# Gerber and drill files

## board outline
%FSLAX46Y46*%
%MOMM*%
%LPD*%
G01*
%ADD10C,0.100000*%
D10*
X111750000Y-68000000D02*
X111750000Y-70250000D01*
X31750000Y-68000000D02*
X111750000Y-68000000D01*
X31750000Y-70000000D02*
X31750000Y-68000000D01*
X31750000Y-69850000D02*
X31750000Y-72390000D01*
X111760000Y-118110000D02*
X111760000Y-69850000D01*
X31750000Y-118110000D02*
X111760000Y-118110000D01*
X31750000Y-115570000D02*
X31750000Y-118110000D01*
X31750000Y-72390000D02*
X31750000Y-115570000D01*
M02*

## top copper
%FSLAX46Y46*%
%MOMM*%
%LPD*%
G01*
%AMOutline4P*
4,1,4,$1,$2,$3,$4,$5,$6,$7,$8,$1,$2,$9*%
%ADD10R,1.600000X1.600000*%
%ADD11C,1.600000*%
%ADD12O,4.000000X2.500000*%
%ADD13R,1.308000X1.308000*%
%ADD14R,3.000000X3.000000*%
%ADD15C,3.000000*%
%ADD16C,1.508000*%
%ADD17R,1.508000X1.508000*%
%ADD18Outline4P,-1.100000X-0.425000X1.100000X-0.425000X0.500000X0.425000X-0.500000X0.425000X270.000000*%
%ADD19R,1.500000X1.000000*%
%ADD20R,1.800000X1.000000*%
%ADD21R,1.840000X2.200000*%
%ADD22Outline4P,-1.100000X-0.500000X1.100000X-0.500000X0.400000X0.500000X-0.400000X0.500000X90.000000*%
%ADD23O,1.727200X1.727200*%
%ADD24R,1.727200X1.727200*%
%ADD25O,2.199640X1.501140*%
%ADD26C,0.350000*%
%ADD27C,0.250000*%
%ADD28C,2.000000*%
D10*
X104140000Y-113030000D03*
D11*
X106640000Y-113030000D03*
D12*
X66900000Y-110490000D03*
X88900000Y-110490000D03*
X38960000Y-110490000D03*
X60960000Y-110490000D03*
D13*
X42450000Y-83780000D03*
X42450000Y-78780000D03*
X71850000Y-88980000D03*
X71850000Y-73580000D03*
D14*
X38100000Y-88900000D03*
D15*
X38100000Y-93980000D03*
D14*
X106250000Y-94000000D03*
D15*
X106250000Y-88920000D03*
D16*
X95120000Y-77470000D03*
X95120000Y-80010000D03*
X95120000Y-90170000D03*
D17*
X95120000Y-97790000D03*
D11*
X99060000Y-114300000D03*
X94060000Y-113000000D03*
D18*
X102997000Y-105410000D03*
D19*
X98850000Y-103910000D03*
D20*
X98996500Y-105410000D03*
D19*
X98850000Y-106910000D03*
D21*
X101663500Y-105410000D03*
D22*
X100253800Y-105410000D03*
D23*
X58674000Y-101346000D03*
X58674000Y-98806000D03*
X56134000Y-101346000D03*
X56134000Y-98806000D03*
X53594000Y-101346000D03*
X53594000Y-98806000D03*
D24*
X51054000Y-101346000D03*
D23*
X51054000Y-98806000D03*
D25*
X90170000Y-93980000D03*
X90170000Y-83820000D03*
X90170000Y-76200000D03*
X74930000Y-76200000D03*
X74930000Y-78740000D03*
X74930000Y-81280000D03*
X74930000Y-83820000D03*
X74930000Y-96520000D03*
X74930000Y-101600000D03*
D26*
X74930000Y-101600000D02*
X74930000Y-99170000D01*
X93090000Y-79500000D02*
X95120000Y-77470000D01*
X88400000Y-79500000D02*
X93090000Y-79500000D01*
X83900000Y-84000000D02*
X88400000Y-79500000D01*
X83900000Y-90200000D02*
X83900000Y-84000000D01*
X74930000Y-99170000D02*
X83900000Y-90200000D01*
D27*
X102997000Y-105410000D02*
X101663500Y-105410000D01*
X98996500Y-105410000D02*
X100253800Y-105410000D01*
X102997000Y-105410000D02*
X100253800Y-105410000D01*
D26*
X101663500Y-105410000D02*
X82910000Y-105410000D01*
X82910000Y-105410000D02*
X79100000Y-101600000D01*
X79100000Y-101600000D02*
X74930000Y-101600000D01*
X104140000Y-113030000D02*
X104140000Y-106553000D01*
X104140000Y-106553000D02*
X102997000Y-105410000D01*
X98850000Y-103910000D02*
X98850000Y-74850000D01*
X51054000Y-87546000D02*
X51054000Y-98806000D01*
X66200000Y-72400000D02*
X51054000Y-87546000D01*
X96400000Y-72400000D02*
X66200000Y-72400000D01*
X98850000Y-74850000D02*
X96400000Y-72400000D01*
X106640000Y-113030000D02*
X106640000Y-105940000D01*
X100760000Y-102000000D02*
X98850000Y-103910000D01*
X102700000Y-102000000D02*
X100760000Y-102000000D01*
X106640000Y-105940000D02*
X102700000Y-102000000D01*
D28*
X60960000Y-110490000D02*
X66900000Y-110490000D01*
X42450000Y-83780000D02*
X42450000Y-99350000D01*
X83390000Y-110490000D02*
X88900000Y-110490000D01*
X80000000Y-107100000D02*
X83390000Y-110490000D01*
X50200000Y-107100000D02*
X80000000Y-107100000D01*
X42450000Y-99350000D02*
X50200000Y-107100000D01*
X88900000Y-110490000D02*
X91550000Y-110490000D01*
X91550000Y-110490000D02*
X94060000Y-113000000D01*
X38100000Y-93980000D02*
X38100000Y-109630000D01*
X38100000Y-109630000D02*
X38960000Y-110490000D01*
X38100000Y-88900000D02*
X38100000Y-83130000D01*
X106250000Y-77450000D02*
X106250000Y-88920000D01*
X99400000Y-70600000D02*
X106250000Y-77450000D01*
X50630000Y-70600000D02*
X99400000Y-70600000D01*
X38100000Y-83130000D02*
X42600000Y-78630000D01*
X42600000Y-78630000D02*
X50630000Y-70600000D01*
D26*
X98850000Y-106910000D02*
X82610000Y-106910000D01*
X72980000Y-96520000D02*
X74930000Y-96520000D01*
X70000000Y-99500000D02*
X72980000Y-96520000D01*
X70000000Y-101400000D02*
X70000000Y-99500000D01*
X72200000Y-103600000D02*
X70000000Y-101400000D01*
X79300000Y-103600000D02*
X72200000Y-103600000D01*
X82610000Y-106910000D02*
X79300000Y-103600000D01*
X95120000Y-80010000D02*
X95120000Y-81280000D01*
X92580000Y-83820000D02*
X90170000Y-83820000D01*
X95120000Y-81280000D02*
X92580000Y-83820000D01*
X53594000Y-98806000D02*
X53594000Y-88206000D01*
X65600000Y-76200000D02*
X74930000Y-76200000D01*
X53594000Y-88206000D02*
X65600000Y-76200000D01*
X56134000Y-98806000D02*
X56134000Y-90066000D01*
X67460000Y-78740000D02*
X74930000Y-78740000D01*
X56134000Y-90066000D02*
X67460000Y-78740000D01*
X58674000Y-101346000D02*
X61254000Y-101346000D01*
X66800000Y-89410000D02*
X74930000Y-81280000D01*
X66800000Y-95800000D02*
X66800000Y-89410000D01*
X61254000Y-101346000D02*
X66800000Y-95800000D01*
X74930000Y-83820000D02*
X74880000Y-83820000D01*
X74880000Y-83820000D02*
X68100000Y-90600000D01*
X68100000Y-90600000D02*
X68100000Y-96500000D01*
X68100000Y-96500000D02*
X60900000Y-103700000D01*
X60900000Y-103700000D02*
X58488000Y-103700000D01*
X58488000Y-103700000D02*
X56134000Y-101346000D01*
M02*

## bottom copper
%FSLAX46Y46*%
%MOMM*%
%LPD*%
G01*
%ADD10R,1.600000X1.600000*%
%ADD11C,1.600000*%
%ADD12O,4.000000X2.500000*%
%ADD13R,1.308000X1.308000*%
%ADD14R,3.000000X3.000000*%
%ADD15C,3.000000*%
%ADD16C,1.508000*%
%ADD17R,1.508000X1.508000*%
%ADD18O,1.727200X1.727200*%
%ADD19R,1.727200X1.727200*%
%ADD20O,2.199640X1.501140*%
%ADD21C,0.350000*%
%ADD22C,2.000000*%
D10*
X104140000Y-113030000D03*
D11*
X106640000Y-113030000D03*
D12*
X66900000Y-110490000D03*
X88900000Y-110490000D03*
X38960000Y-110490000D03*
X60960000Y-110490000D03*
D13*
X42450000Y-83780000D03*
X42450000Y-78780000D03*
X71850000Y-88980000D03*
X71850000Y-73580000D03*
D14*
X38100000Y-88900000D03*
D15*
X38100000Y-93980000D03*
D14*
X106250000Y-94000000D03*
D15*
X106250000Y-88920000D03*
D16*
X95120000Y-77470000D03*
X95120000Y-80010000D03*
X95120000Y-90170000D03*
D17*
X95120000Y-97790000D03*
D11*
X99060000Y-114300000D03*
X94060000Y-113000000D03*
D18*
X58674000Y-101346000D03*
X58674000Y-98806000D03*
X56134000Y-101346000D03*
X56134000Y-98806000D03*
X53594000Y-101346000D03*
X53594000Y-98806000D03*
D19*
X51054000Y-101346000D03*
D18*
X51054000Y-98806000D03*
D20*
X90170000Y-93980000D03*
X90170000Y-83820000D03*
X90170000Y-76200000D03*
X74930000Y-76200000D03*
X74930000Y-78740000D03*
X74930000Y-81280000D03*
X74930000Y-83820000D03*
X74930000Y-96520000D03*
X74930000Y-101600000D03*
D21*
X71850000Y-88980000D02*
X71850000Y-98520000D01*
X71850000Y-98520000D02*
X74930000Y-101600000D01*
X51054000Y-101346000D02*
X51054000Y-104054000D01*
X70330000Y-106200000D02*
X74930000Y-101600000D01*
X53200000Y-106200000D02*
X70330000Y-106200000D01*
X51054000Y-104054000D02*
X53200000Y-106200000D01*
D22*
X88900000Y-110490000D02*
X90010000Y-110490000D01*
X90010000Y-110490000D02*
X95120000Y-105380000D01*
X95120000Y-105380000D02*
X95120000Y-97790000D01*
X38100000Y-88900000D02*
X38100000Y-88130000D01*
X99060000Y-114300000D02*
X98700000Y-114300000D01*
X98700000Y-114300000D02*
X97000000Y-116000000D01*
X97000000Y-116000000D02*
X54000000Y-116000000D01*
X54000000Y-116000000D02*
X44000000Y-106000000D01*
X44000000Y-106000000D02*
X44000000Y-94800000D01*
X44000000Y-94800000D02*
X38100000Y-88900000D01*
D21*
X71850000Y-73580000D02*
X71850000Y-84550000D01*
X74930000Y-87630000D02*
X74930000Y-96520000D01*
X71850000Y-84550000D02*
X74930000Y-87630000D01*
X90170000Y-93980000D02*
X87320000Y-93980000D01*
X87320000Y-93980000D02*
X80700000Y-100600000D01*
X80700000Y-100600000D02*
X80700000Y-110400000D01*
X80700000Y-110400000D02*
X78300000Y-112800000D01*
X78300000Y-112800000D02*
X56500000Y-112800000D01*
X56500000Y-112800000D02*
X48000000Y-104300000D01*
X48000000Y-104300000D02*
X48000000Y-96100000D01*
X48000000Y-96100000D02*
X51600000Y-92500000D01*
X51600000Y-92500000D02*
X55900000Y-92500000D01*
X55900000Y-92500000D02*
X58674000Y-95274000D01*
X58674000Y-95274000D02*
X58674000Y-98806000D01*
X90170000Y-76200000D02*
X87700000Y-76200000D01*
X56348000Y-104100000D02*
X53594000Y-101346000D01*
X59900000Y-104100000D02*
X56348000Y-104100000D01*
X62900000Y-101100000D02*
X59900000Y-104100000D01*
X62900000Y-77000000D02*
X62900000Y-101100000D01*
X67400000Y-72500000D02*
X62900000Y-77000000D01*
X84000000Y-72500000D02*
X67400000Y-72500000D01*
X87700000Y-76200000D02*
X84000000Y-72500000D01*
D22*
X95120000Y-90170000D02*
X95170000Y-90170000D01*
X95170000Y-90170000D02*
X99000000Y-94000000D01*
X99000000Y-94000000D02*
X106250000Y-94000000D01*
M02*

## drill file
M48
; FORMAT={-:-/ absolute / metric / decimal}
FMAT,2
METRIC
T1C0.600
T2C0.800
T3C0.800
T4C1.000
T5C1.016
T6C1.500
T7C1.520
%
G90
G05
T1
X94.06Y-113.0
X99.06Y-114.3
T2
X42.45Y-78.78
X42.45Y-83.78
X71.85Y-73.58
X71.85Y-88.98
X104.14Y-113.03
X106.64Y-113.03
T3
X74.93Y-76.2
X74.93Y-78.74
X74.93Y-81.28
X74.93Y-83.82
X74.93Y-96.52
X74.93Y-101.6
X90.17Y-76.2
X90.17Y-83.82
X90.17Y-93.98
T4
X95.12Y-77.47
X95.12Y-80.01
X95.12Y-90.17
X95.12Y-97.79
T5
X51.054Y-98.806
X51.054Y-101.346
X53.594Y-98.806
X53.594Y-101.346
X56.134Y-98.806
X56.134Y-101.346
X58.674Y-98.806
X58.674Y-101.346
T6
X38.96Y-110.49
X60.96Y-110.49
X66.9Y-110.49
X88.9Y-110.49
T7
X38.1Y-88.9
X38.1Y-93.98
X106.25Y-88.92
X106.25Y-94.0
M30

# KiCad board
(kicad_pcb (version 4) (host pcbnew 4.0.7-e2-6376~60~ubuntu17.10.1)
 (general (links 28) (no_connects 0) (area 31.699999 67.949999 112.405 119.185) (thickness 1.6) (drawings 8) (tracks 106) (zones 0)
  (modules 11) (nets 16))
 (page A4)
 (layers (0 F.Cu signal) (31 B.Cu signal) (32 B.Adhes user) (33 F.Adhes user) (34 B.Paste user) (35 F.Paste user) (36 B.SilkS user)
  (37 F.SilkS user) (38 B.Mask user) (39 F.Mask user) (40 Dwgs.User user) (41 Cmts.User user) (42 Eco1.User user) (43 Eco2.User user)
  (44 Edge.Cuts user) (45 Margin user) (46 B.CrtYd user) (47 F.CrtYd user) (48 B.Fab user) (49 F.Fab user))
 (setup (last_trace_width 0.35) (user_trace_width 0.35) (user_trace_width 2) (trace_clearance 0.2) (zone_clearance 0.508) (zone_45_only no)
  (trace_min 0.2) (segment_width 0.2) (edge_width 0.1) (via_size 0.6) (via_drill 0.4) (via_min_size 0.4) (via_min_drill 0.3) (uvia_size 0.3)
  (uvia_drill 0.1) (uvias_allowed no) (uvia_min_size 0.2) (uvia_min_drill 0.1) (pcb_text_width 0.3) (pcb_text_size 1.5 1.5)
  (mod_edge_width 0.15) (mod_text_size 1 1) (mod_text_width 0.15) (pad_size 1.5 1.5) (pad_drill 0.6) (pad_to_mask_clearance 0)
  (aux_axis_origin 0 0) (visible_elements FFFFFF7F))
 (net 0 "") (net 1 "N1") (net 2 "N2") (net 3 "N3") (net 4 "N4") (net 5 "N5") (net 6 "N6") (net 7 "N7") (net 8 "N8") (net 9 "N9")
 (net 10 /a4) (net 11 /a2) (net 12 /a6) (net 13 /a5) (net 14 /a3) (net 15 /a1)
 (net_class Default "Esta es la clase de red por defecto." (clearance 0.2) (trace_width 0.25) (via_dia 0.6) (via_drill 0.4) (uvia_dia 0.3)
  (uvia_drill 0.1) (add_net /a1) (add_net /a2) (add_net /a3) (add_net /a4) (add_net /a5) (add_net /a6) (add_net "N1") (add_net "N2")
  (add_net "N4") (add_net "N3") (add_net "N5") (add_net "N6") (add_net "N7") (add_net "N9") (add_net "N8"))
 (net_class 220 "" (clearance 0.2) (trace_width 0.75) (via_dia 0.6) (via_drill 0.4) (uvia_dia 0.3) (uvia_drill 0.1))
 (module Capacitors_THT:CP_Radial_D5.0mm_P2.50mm (layer F.Cu) (at 104.14 113.03)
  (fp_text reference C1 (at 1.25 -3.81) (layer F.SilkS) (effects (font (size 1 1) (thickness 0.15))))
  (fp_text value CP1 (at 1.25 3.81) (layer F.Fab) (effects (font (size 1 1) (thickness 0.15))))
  (pad 1 thru_hole rect (at 0 0) (size 1.6 1.6) (drill 0.8) (layers *.Cu *.Mask) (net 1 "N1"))
  (pad 2 thru_hole circle (at 2.5 0) (size 1.6 1.6) (drill 0.8) (layers *.Cu *.Mask) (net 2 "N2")))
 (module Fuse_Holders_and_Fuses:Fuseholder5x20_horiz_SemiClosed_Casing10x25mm (layer F.Cu) (at 88.9 110.49 180)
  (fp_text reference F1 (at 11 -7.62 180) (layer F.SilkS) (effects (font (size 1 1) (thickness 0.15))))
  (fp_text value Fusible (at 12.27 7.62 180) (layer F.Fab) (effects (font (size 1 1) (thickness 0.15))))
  (pad 2 thru_hole oval (at 22 0 90) (size 2.5 4) (drill 1.5) (layers *.Cu *.Mask) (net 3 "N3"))
  (pad 1 thru_hole oval (at 0 0 90) (size 2.5 4) (drill 1.5) (layers *.Cu *.Mask) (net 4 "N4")))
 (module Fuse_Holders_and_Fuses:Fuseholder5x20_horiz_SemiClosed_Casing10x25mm (layer F.Cu) (at 60.96 110.49 180)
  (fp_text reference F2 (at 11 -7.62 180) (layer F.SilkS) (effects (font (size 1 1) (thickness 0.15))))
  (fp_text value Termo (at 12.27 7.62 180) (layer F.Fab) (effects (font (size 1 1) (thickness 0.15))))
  (pad 2 thru_hole oval (at 22 0 90) (size 2.5 4) (drill 1.5) (layers *.Cu *.Mask) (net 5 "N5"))
  (pad 1 thru_hole oval (at 0 0 90) (size 2.5 4) (drill 1.5) (layers *.Cu *.Mask) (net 3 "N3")))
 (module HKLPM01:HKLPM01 (layer B.Cu) (at 57.15 81.28)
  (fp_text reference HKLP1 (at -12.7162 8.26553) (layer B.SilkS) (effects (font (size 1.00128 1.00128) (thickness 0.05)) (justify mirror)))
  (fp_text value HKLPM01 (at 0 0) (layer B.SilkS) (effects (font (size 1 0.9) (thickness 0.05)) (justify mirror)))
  (pad P$1 thru_hole rect (at -14.7 2.5) (size 1.308 1.308) (drill 0.8) (layers *.Cu *.Mask B.SilkS) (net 4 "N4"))
  (pad P$2 thru_hole rect (at -14.7 -2.5) (size 1.308 1.308) (drill 0.8) (layers *.Cu *.Mask B.SilkS) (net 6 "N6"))
  (pad P$3 thru_hole rect (at 14.7 7.7) (size 1.308 1.308) (drill 0.8) (layers *.Cu *.Mask B.SilkS) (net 1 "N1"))
  (pad P$4 thru_hole rect (at 14.7 -7.7) (size 1.308 1.308) (drill 0.8) (layers *.Cu *.Mask B.SilkS) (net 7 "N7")))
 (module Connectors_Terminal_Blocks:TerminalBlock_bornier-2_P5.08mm (layer F.Cu) (at 38.1 88.9 270)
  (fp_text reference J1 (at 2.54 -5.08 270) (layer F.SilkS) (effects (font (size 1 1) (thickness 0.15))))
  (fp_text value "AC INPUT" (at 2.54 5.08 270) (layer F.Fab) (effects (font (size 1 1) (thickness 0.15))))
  (pad 1 thru_hole rect (at 0 0 270) (size 3 3) (drill 1.52) (layers *.Cu *.Mask) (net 6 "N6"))
  (pad 2 thru_hole circle (at 5.08 0 270) (size 3 3) (drill 1.52) (layers *.Cu *.Mask) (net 5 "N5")))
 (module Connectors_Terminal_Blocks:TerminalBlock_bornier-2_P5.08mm (layer F.Cu) (at 106.25 94 90)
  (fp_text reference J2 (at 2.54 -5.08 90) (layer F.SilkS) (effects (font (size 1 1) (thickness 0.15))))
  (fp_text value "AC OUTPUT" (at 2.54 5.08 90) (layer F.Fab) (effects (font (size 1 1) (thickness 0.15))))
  (pad 1 thru_hole rect (at 0 0 90) (size 3 3) (drill 1.52) (layers *.Cu *.Mask) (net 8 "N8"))
  (pad 2 thru_hole circle (at 5.08 0 90) (size 3 3) (drill 1.52) (layers *.Cu *.Mask) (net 6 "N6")))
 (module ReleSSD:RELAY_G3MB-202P (layer F.Cu) (at 96.52 87.63 270)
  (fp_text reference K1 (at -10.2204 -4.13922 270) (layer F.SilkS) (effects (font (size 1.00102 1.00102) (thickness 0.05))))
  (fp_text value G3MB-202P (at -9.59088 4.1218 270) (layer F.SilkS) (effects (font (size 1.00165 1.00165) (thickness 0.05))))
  (pad 4 thru_hole circle (at -10.16 1.4 270) (size 1.508 1.508) (drill 1) (layers *.Cu *.Mask F.SilkS) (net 1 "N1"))
  (pad 3 thru_hole circle (at -7.62 1.4 270) (size 1.508 1.508) (drill 1) (layers *.Cu *.Mask F.SilkS) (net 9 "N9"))
  (pad 2 thru_hole circle (at 2.54 1.4 270) (size 1.508 1.508) (drill 1) (layers *.Cu *.Mask F.SilkS) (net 8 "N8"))
  (pad 1 thru_hole rect (at 10.16 1.4 270) (size 1.508 1.508) (drill 1) (layers *.Cu *.Mask F.SilkS) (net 4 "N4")))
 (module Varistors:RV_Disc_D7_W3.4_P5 (layer F.Cu) (at 99.06 114.3 180)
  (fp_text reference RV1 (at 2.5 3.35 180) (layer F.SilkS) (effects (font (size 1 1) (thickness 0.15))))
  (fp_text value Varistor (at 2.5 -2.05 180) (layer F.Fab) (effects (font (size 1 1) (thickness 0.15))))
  (pad 1 thru_hole circle (at 0 0 180) (size 1.6 1.6) (drill 0.6) (layers *.Cu *.Mask) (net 6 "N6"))
  (pad 2 thru_hole circle (at 5 1.3 180) (size 1.6 1.6) (drill 0.6) (layers *.Cu *.Mask) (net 4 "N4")))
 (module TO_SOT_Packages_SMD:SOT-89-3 (layer F.Cu) (at 100.33 105.41)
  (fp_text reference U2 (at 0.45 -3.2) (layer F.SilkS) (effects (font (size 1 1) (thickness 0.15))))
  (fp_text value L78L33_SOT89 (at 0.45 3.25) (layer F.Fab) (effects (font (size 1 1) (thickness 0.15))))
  (pad 2 smd trapezoid (at 2.667 0 270) (size 1.6 0.85) (rect_delta 0 0.6) (layers F.Cu F.Paste F.Mask) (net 1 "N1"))
  (pad 1 smd rect (at -1.48 -1.5 270) (size 1 1.5) (layers F.Cu F.Paste F.Mask) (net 2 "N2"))
  (pad 2 smd rect (at -1.3335 0 270) (size 1 1.8) (layers F.Cu F.Paste F.Mask) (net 1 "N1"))
  (pad 3 smd rect (at -1.48 1.5 270) (size 1 1.5) (layers F.Cu F.Paste F.Mask) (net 7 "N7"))
  (pad 2 smd rect (at 1.3335 0 270) (size 2.2 1.84) (layers F.Cu F.Paste F.Mask) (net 1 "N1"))
  (pad 2 smd trapezoid (at -0.0762 0 90) (size 1.5 1) (rect_delta 0 0.7) (layers F.Cu F.Paste F.Mask) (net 1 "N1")))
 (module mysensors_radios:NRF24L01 (layer F.Cu) (at 49.53 102.87 180)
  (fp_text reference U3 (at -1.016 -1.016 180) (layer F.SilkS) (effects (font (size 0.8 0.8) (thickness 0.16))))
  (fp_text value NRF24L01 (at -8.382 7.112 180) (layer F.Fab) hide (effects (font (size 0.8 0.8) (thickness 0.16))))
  (pad 7 thru_hole oval (at -9.144 1.524 180) (size 1.7272 1.7272) (drill 1.016) (layers *.Cu *.Mask F.SilkS) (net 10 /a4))
  (pad 8 thru_hole oval (at -9.144 4.064 180) (size 1.7272 1.7272) (drill 1.016) (layers *.Cu *.Mask F.SilkS) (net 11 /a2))
  (pad 5 thru_hole oval (at -6.604 1.524 180) (size 1.7272 1.7272) (drill 1.016) (layers *.Cu *.Mask F.SilkS) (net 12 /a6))
  (pad 6 thru_hole oval (at -6.604 4.064 180) (size 1.7272 1.7272) (drill 1.016) (layers *.Cu *.Mask F.SilkS) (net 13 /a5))
  (pad 3 thru_hole oval (at -4.064 1.524 180) (size 1.7272 1.7272) (drill 1.016) (layers *.Cu *.Mask F.SilkS) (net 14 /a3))
  (pad 4 thru_hole oval (at -4.064 4.064 180) (size 1.7272 1.7272) (drill 1.016) (layers *.Cu *.Mask F.SilkS) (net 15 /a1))
  (pad 1 thru_hole rect (at -1.524 1.524 180) (size 1.7272 1.7272) (drill 1.016) (layers *.Cu *.Mask F.SilkS) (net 1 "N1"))
  (pad 2 thru_hole oval (at -1.524 4.064 180) (size 1.7272 1.7272) (drill 1.016) (layers *.Cu *.Mask F.SilkS) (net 2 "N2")))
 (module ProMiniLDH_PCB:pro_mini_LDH (layer F.Cu) (at 82.55 90.17 90)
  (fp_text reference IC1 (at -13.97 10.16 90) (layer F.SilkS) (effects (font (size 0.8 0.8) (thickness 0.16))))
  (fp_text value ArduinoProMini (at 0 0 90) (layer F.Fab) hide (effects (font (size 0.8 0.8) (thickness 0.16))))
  (pad 5 thru_hole oval (at -3.81 7.62 90) (size 1.50114 2.19964) (drill 0.8001) (layers *.Cu *.Mask F.SilkS) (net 11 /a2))
  (pad 9 thru_hole oval (at 6.35 7.62 90) (size 1.50114 2.19964) (drill 0.8001) (layers *.Cu *.Mask F.SilkS) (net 9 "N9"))
  (pad 12 thru_hole oval (at 13.97 7.62 90) (size 1.50114 2.19964) (drill 0.8001) (layers *.Cu *.Mask F.SilkS) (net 14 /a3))
  (pad 13 thru_hole oval (at 13.97 -7.62 90) (size 1.50114 2.19964) (drill 0.8001) (layers *.Cu *.Mask F.SilkS) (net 15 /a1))
  (pad 14 thru_hole oval (at 11.43 -7.62 90) (size 1.50114 2.19964) (drill 0.8001) (layers *.Cu *.Mask F.SilkS) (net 13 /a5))
  (pad 15 thru_hole oval (at 8.89 -7.62 90) (size 1.50114 2.19964) (drill 0.8001) (layers *.Cu *.Mask F.SilkS) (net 10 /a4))
  (pad 16 thru_hole oval (at 6.35 -7.62 90) (size 1.50114 2.19964) (drill 0.8001) (layers *.Cu *.Mask F.SilkS) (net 12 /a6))
  (pad 21 thru_hole oval (at -6.35 -7.62 90) (size 1.50114 2.19964) (drill 0.8001) (layers *.Cu *.Mask F.SilkS) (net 7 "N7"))
  (pad 23 thru_hole oval (at -11.43 -7.62 90) (size 1.50114 2.19964) (drill 0.8001) (layers *.Cu *.Mask F.SilkS) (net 1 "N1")))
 (gr_line (start 111.75 68) (end 111.75 70.25) (angle 90) (layer Edge.Cuts) (width 0.1))
 (gr_line (start 31.75 68) (end 111.75 68) (angle 90) (layer Edge.Cuts) (width 0.1))
 (gr_line (start 31.75 70) (end 31.75 68) (angle 90) (layer Edge.Cuts) (width 0.1))
 (gr_line (start 31.75 69.85) (end 31.75 72.39) (angle 90) (layer Edge.Cuts) (width 0.1))
 (gr_line (start 111.76 118.11) (end 111.76 69.85) (angle 90) (layer Edge.Cuts) (width 0.1))
 (gr_line (start 31.75 118.11) (end 111.76 118.11) (angle 90) (layer Edge.Cuts) (width 0.1))
 (gr_line (start 31.75 115.57) (end 31.75 118.11) (angle 90) (layer Edge.Cuts) (width 0.1))
 (gr_line (start 31.75 72.39) (end 31.75 115.57) (angle 90) (layer Edge.Cuts) (width 0.1))
 (segment (start 74.93 101.6) (end 74.93 99.17) (width 0.35) (layer F.Cu) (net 1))
 (segment (start 93.09 79.5) (end 95.12 77.47) (width 0.35) (layer F.Cu) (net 1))
 (segment (start 88.4 79.5) (end 93.09 79.5) (width 0.35) (layer F.Cu) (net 1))
 (segment (start 83.9 84) (end 88.4 79.5) (width 0.35) (layer F.Cu) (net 1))
 (segment (start 83.9 90.2) (end 83.9 84) (width 0.35) (layer F.Cu) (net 1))
 (segment (start 74.93 99.17) (end 83.9 90.2) (width 0.35) (layer F.Cu) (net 1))
 (segment (start 71.85 88.98) (end 71.85 98.52) (width 0.35) (layer B.Cu) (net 1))
 (segment (start 71.85 98.52) (end 74.93 101.6) (width 0.35) (layer B.Cu) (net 1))
 (segment (start 102.997 105.41) (end 101.6635 105.41) (width 0.25) (layer F.Cu) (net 1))
 (segment (start 98.9965 105.41) (end 100.2538 105.41) (width 0.25) (layer F.Cu) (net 1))
 (segment (start 102.997 105.41) (end 100.2538 105.41) (width 0.25) (layer F.Cu) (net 1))
 (segment (start 51.054 101.346) (end 51.054 104.054) (width 0.35) (layer B.Cu) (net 1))
 (segment (start 70.33 106.2) (end 74.93 101.6) (width 0.35) (layer B.Cu) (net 1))
 (segment (start 53.2 106.2) (end 70.33 106.2) (width 0.35) (layer B.Cu) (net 1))
 (segment (start 51.054 104.054) (end 53.2 106.2) (width 0.35) (layer B.Cu) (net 1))
 (segment (start 101.6635 105.41) (end 82.91 105.41) (width 0.35) (layer F.Cu) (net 1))
 (segment (start 82.91 105.41) (end 79.1 101.6) (width 0.35) (layer F.Cu) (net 1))
 (segment (start 79.1 101.6) (end 74.93 101.6) (width 0.35) (layer F.Cu) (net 1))
 (segment (start 104.14 113.03) (end 104.14 106.553) (width 0.35) (layer F.Cu) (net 1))
 (segment (start 104.14 106.553) (end 102.997 105.41) (width 0.35) (layer F.Cu) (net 1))
 (segment (start 98.85 103.91) (end 98.85 74.85) (width 0.35) (layer F.Cu) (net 2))
 (segment (start 51.054 87.546) (end 51.054 98.806) (width 0.35) (layer F.Cu) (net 2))
 (segment (start 66.2 72.4) (end 51.054 87.546) (width 0.35) (layer F.Cu) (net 2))
 (segment (start 96.4 72.4) (end 66.2 72.4) (width 0.35) (layer F.Cu) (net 2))
 (segment (start 98.85 74.85) (end 96.4 72.4) (width 0.35) (layer F.Cu) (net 2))
 (segment (start 106.64 113.03) (end 106.64 105.94) (width 0.35) (layer F.Cu) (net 2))
 (segment (start 100.76 102) (end 98.85 103.91) (width 0.35) (layer F.Cu) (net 2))
 (segment (start 102.7 102) (end 100.76 102) (width 0.35) (layer F.Cu) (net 2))
 (segment (start 106.64 105.94) (end 102.7 102) (width 0.35) (layer F.Cu) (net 2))
 (segment (start 60.96 110.49) (end 66.9 110.49) (width 2) (layer F.Cu) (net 3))
 (segment (start 42.45 83.78) (end 42.45 99.35) (width 2) (layer F.Cu) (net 4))
 (segment (start 83.39 110.49) (end 88.9 110.49) (width 2) (layer F.Cu) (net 4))
 (segment (start 80 107.1) (end 83.39 110.49) (width 2) (layer F.Cu) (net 4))
 (segment (start 50.2 107.1) (end 80 107.1) (width 2) (layer F.Cu) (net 4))
 (segment (start 42.45 99.35) (end 50.2 107.1) (width 2) (layer F.Cu) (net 4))
 (segment (start 88.9 110.49) (end 90.01 110.49) (width 2) (layer B.Cu) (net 4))
 (segment (start 90.01 110.49) (end 95.12 105.38) (width 2) (layer B.Cu) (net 4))
 (segment (start 95.12 105.38) (end 95.12 97.79) (width 2) (layer B.Cu) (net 4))
 (segment (start 88.9 110.49) (end 91.55 110.49) (width 2) (layer F.Cu) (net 4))
 (segment (start 91.55 110.49) (end 94.06 113) (width 2) (layer F.Cu) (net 4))
 (segment (start 38.1 93.98) (end 38.1 109.63) (width 2) (layer F.Cu) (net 5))
 (segment (start 38.1 109.63) (end 38.96 110.49) (width 2) (layer F.Cu) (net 5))
 (segment (start 38.1 88.9) (end 38.1 83.13) (width 2) (layer F.Cu) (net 6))
 (segment (start 106.25 77.45) (end 106.25 88.92) (width 2) (layer F.Cu) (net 6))
 (segment (start 99.4 70.6) (end 106.25 77.45) (width 2) (layer F.Cu) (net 6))
 (segment (start 50.63 70.6) (end 99.4 70.6) (width 2) (layer F.Cu) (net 6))
 (segment (start 38.1 83.13) (end 42.6 78.63) (width 2) (layer F.Cu) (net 6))
 (segment (start 42.6 78.63) (end 50.63 70.6) (width 2) (layer F.Cu) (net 6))
 (segment (start 38.1 88.9) (end 38.1 88.13) (width 2) (layer B.Cu) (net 6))
 (segment (start 99.06 114.3) (end 98.7 114.3) (width 2) (layer B.Cu) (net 6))
 (segment (start 98.7 114.3) (end 97 116) (width 2) (layer B.Cu) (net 6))
 (segment (start 97 116) (end 54 116) (width 2) (layer B.Cu) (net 6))
 (segment (start 54 116) (end 44 106) (width 2) (layer B.Cu) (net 6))
 (segment (start 44 106) (end 44 94.8) (width 2) (layer B.Cu) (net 6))
 (segment (start 44 94.8) (end 38.1 88.9) (width 2) (layer B.Cu) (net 6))
 (segment (start 98.85 106.91) (end 82.61 106.91) (width 0.35) (layer F.Cu) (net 7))
 (segment (start 72.98 96.52) (end 74.93 96.52) (width 0.35) (layer F.Cu) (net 7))
 (segment (start 70 99.5) (end 72.98 96.52) (width 0.35) (layer F.Cu) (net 7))
 (segment (start 70 101.4) (end 70 99.5) (width 0.35) (layer F.Cu) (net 7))
 (segment (start 72.2 103.6) (end 70 101.4) (width 0.35) (layer F.Cu) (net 7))
 (segment (start 79.3 103.6) (end 72.2 103.6) (width 0.35) (layer F.Cu) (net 7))
 (segment (start 82.61 106.91) (end 79.3 103.6) (width 0.35) (layer F.Cu) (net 7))
 (segment (start 71.85 73.58) (end 71.85 84.55) (width 0.35) (layer B.Cu) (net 7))
 (segment (start 74.93 87.63) (end 74.93 96.52) (width 0.35) (layer B.Cu) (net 7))
 (segment (start 71.85 84.55) (end 74.93 87.63) (width 0.35) (layer B.Cu) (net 7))
 (segment (start 90.17 93.98) (end 87.32 93.98) (width 0.35) (layer B.Cu) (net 11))
 (segment (start 87.32 93.98) (end 80.7 100.6) (width 0.35) (layer B.Cu) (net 11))
 (segment (start 80.7 100.6) (end 80.7 110.4) (width 0.35) (layer B.Cu) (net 11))
 (segment (start 80.7 110.4) (end 78.3 112.8) (width 0.35) (layer B.Cu) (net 11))
 (segment (start 78.3 112.8) (end 56.5 112.8) (width 0.35) (layer B.Cu) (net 11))
 (segment (start 56.5 112.8) (end 48 104.3) (width 0.35) (layer B.Cu) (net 11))
 (segment (start 48 104.3) (end 48 96.1) (width 0.35) (layer B.Cu) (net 11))
 (segment (start 48 96.1) (end 51.6 92.5) (width 0.35) (layer B.Cu) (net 11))
 (segment (start 51.6 92.5) (end 55.9 92.5) (width 0.35) (layer B.Cu) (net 11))
 (segment (start 55.9 92.5) (end 58.674 95.274) (width 0.35) (layer B.Cu) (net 11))
 (segment (start 58.674 95.274) (end 58.674 98.806) (width 0.35) (layer B.Cu) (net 11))
 (segment (start 95.12 80.01) (end 95.12 81.28) (width 0.35) (layer F.Cu) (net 9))
 (segment (start 92.58 83.82) (end 90.17 83.82) (width 0.35) (layer F.Cu) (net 9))
 (segment (start 95.12 81.28) (end 92.58 83.82) (width 0.35) (layer F.Cu) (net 9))
 (segment (start 90.17 76.2) (end 87.7 76.2) (width 0.35) (layer B.Cu) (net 14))
 (segment (start 56.348 104.1) (end 53.594 101.346) (width 0.35) (layer B.Cu) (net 14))
 (segment (start 59.9 104.1) (end 56.348 104.1) (width 0.35) (layer B.Cu) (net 14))
 (segment (start 62.9 101.1) (end 59.9 104.1) (width 0.35) (layer B.Cu) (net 14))
 (segment (start 62.9 77) (end 62.9 101.1) (width 0.35) (layer B.Cu) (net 14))
 (segment (start 67.4 72.5) (end 62.9 77) (width 0.35) (layer B.Cu) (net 14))
 (segment (start 84 72.5) (end 67.4 72.5) (width 0.35) (layer B.Cu) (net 14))
 (segment (start 87.7 76.2) (end 84 72.5) (width 0.35) (layer B.Cu) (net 14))
 (segment (start 53.594 98.806) (end 53.594 88.206) (width 0.35) (layer F.Cu) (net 15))
 (segment (start 65.6 76.2) (end 74.93 76.2) (width 0.35) (layer F.Cu) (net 15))
 (segment (start 53.594 88.206) (end 65.6 76.2) (width 0.35) (layer F.Cu) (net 15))
 (segment (start 56.134 98.806) (end 56.134 90.066) (width 0.35) (layer F.Cu) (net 13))
 (segment (start 67.46 78.74) (end 74.93 78.74) (width 0.35) (layer F.Cu) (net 13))
 (segment (start 56.134 90.066) (end 67.46 78.74) (width 0.35) (layer F.Cu) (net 13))
 (segment (start 58.674 101.346) (end 61.254 101.346) (width 0.35) (layer F.Cu) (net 10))
 (segment (start 66.8 89.41) (end 74.93 81.28) (width 0.35) (layer F.Cu) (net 10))
 (segment (start 66.8 95.8) (end 66.8 89.41) (width 0.35) (layer F.Cu) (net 10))
 (segment (start 61.254 101.346) (end 66.8 95.8) (width 0.35) (layer F.Cu) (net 10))
 (segment (start 74.93 83.82) (end 74.88 83.82) (width 0.35) (layer F.Cu) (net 12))
 (segment (start 74.88 83.82) (end 68.1 90.6) (width 0.35) (layer F.Cu) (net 12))
 (segment (start 68.1 90.6) (end 68.1 96.5) (width 0.35) (layer F.Cu) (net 12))
 (segment (start 68.1 96.5) (end 60.9 103.7) (width 0.35) (layer F.Cu) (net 12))
 (segment (start 60.9 103.7) (end 58.488 103.7) (width 0.35) (layer F.Cu) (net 12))
 (segment (start 58.488 103.7) (end 56.134 101.346) (width 0.35) (layer F.Cu) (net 12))
 (segment (start 95.12 90.17) (end 95.17 90.17) (width 2) (layer B.Cu) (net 8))
 (segment (start 95.17 90.17) (end 99 94) (width 2) (layer B.Cu) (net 8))
 (segment (start 99 94) (end 106.25 94) (width 2) (layer B.Cu) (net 8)))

